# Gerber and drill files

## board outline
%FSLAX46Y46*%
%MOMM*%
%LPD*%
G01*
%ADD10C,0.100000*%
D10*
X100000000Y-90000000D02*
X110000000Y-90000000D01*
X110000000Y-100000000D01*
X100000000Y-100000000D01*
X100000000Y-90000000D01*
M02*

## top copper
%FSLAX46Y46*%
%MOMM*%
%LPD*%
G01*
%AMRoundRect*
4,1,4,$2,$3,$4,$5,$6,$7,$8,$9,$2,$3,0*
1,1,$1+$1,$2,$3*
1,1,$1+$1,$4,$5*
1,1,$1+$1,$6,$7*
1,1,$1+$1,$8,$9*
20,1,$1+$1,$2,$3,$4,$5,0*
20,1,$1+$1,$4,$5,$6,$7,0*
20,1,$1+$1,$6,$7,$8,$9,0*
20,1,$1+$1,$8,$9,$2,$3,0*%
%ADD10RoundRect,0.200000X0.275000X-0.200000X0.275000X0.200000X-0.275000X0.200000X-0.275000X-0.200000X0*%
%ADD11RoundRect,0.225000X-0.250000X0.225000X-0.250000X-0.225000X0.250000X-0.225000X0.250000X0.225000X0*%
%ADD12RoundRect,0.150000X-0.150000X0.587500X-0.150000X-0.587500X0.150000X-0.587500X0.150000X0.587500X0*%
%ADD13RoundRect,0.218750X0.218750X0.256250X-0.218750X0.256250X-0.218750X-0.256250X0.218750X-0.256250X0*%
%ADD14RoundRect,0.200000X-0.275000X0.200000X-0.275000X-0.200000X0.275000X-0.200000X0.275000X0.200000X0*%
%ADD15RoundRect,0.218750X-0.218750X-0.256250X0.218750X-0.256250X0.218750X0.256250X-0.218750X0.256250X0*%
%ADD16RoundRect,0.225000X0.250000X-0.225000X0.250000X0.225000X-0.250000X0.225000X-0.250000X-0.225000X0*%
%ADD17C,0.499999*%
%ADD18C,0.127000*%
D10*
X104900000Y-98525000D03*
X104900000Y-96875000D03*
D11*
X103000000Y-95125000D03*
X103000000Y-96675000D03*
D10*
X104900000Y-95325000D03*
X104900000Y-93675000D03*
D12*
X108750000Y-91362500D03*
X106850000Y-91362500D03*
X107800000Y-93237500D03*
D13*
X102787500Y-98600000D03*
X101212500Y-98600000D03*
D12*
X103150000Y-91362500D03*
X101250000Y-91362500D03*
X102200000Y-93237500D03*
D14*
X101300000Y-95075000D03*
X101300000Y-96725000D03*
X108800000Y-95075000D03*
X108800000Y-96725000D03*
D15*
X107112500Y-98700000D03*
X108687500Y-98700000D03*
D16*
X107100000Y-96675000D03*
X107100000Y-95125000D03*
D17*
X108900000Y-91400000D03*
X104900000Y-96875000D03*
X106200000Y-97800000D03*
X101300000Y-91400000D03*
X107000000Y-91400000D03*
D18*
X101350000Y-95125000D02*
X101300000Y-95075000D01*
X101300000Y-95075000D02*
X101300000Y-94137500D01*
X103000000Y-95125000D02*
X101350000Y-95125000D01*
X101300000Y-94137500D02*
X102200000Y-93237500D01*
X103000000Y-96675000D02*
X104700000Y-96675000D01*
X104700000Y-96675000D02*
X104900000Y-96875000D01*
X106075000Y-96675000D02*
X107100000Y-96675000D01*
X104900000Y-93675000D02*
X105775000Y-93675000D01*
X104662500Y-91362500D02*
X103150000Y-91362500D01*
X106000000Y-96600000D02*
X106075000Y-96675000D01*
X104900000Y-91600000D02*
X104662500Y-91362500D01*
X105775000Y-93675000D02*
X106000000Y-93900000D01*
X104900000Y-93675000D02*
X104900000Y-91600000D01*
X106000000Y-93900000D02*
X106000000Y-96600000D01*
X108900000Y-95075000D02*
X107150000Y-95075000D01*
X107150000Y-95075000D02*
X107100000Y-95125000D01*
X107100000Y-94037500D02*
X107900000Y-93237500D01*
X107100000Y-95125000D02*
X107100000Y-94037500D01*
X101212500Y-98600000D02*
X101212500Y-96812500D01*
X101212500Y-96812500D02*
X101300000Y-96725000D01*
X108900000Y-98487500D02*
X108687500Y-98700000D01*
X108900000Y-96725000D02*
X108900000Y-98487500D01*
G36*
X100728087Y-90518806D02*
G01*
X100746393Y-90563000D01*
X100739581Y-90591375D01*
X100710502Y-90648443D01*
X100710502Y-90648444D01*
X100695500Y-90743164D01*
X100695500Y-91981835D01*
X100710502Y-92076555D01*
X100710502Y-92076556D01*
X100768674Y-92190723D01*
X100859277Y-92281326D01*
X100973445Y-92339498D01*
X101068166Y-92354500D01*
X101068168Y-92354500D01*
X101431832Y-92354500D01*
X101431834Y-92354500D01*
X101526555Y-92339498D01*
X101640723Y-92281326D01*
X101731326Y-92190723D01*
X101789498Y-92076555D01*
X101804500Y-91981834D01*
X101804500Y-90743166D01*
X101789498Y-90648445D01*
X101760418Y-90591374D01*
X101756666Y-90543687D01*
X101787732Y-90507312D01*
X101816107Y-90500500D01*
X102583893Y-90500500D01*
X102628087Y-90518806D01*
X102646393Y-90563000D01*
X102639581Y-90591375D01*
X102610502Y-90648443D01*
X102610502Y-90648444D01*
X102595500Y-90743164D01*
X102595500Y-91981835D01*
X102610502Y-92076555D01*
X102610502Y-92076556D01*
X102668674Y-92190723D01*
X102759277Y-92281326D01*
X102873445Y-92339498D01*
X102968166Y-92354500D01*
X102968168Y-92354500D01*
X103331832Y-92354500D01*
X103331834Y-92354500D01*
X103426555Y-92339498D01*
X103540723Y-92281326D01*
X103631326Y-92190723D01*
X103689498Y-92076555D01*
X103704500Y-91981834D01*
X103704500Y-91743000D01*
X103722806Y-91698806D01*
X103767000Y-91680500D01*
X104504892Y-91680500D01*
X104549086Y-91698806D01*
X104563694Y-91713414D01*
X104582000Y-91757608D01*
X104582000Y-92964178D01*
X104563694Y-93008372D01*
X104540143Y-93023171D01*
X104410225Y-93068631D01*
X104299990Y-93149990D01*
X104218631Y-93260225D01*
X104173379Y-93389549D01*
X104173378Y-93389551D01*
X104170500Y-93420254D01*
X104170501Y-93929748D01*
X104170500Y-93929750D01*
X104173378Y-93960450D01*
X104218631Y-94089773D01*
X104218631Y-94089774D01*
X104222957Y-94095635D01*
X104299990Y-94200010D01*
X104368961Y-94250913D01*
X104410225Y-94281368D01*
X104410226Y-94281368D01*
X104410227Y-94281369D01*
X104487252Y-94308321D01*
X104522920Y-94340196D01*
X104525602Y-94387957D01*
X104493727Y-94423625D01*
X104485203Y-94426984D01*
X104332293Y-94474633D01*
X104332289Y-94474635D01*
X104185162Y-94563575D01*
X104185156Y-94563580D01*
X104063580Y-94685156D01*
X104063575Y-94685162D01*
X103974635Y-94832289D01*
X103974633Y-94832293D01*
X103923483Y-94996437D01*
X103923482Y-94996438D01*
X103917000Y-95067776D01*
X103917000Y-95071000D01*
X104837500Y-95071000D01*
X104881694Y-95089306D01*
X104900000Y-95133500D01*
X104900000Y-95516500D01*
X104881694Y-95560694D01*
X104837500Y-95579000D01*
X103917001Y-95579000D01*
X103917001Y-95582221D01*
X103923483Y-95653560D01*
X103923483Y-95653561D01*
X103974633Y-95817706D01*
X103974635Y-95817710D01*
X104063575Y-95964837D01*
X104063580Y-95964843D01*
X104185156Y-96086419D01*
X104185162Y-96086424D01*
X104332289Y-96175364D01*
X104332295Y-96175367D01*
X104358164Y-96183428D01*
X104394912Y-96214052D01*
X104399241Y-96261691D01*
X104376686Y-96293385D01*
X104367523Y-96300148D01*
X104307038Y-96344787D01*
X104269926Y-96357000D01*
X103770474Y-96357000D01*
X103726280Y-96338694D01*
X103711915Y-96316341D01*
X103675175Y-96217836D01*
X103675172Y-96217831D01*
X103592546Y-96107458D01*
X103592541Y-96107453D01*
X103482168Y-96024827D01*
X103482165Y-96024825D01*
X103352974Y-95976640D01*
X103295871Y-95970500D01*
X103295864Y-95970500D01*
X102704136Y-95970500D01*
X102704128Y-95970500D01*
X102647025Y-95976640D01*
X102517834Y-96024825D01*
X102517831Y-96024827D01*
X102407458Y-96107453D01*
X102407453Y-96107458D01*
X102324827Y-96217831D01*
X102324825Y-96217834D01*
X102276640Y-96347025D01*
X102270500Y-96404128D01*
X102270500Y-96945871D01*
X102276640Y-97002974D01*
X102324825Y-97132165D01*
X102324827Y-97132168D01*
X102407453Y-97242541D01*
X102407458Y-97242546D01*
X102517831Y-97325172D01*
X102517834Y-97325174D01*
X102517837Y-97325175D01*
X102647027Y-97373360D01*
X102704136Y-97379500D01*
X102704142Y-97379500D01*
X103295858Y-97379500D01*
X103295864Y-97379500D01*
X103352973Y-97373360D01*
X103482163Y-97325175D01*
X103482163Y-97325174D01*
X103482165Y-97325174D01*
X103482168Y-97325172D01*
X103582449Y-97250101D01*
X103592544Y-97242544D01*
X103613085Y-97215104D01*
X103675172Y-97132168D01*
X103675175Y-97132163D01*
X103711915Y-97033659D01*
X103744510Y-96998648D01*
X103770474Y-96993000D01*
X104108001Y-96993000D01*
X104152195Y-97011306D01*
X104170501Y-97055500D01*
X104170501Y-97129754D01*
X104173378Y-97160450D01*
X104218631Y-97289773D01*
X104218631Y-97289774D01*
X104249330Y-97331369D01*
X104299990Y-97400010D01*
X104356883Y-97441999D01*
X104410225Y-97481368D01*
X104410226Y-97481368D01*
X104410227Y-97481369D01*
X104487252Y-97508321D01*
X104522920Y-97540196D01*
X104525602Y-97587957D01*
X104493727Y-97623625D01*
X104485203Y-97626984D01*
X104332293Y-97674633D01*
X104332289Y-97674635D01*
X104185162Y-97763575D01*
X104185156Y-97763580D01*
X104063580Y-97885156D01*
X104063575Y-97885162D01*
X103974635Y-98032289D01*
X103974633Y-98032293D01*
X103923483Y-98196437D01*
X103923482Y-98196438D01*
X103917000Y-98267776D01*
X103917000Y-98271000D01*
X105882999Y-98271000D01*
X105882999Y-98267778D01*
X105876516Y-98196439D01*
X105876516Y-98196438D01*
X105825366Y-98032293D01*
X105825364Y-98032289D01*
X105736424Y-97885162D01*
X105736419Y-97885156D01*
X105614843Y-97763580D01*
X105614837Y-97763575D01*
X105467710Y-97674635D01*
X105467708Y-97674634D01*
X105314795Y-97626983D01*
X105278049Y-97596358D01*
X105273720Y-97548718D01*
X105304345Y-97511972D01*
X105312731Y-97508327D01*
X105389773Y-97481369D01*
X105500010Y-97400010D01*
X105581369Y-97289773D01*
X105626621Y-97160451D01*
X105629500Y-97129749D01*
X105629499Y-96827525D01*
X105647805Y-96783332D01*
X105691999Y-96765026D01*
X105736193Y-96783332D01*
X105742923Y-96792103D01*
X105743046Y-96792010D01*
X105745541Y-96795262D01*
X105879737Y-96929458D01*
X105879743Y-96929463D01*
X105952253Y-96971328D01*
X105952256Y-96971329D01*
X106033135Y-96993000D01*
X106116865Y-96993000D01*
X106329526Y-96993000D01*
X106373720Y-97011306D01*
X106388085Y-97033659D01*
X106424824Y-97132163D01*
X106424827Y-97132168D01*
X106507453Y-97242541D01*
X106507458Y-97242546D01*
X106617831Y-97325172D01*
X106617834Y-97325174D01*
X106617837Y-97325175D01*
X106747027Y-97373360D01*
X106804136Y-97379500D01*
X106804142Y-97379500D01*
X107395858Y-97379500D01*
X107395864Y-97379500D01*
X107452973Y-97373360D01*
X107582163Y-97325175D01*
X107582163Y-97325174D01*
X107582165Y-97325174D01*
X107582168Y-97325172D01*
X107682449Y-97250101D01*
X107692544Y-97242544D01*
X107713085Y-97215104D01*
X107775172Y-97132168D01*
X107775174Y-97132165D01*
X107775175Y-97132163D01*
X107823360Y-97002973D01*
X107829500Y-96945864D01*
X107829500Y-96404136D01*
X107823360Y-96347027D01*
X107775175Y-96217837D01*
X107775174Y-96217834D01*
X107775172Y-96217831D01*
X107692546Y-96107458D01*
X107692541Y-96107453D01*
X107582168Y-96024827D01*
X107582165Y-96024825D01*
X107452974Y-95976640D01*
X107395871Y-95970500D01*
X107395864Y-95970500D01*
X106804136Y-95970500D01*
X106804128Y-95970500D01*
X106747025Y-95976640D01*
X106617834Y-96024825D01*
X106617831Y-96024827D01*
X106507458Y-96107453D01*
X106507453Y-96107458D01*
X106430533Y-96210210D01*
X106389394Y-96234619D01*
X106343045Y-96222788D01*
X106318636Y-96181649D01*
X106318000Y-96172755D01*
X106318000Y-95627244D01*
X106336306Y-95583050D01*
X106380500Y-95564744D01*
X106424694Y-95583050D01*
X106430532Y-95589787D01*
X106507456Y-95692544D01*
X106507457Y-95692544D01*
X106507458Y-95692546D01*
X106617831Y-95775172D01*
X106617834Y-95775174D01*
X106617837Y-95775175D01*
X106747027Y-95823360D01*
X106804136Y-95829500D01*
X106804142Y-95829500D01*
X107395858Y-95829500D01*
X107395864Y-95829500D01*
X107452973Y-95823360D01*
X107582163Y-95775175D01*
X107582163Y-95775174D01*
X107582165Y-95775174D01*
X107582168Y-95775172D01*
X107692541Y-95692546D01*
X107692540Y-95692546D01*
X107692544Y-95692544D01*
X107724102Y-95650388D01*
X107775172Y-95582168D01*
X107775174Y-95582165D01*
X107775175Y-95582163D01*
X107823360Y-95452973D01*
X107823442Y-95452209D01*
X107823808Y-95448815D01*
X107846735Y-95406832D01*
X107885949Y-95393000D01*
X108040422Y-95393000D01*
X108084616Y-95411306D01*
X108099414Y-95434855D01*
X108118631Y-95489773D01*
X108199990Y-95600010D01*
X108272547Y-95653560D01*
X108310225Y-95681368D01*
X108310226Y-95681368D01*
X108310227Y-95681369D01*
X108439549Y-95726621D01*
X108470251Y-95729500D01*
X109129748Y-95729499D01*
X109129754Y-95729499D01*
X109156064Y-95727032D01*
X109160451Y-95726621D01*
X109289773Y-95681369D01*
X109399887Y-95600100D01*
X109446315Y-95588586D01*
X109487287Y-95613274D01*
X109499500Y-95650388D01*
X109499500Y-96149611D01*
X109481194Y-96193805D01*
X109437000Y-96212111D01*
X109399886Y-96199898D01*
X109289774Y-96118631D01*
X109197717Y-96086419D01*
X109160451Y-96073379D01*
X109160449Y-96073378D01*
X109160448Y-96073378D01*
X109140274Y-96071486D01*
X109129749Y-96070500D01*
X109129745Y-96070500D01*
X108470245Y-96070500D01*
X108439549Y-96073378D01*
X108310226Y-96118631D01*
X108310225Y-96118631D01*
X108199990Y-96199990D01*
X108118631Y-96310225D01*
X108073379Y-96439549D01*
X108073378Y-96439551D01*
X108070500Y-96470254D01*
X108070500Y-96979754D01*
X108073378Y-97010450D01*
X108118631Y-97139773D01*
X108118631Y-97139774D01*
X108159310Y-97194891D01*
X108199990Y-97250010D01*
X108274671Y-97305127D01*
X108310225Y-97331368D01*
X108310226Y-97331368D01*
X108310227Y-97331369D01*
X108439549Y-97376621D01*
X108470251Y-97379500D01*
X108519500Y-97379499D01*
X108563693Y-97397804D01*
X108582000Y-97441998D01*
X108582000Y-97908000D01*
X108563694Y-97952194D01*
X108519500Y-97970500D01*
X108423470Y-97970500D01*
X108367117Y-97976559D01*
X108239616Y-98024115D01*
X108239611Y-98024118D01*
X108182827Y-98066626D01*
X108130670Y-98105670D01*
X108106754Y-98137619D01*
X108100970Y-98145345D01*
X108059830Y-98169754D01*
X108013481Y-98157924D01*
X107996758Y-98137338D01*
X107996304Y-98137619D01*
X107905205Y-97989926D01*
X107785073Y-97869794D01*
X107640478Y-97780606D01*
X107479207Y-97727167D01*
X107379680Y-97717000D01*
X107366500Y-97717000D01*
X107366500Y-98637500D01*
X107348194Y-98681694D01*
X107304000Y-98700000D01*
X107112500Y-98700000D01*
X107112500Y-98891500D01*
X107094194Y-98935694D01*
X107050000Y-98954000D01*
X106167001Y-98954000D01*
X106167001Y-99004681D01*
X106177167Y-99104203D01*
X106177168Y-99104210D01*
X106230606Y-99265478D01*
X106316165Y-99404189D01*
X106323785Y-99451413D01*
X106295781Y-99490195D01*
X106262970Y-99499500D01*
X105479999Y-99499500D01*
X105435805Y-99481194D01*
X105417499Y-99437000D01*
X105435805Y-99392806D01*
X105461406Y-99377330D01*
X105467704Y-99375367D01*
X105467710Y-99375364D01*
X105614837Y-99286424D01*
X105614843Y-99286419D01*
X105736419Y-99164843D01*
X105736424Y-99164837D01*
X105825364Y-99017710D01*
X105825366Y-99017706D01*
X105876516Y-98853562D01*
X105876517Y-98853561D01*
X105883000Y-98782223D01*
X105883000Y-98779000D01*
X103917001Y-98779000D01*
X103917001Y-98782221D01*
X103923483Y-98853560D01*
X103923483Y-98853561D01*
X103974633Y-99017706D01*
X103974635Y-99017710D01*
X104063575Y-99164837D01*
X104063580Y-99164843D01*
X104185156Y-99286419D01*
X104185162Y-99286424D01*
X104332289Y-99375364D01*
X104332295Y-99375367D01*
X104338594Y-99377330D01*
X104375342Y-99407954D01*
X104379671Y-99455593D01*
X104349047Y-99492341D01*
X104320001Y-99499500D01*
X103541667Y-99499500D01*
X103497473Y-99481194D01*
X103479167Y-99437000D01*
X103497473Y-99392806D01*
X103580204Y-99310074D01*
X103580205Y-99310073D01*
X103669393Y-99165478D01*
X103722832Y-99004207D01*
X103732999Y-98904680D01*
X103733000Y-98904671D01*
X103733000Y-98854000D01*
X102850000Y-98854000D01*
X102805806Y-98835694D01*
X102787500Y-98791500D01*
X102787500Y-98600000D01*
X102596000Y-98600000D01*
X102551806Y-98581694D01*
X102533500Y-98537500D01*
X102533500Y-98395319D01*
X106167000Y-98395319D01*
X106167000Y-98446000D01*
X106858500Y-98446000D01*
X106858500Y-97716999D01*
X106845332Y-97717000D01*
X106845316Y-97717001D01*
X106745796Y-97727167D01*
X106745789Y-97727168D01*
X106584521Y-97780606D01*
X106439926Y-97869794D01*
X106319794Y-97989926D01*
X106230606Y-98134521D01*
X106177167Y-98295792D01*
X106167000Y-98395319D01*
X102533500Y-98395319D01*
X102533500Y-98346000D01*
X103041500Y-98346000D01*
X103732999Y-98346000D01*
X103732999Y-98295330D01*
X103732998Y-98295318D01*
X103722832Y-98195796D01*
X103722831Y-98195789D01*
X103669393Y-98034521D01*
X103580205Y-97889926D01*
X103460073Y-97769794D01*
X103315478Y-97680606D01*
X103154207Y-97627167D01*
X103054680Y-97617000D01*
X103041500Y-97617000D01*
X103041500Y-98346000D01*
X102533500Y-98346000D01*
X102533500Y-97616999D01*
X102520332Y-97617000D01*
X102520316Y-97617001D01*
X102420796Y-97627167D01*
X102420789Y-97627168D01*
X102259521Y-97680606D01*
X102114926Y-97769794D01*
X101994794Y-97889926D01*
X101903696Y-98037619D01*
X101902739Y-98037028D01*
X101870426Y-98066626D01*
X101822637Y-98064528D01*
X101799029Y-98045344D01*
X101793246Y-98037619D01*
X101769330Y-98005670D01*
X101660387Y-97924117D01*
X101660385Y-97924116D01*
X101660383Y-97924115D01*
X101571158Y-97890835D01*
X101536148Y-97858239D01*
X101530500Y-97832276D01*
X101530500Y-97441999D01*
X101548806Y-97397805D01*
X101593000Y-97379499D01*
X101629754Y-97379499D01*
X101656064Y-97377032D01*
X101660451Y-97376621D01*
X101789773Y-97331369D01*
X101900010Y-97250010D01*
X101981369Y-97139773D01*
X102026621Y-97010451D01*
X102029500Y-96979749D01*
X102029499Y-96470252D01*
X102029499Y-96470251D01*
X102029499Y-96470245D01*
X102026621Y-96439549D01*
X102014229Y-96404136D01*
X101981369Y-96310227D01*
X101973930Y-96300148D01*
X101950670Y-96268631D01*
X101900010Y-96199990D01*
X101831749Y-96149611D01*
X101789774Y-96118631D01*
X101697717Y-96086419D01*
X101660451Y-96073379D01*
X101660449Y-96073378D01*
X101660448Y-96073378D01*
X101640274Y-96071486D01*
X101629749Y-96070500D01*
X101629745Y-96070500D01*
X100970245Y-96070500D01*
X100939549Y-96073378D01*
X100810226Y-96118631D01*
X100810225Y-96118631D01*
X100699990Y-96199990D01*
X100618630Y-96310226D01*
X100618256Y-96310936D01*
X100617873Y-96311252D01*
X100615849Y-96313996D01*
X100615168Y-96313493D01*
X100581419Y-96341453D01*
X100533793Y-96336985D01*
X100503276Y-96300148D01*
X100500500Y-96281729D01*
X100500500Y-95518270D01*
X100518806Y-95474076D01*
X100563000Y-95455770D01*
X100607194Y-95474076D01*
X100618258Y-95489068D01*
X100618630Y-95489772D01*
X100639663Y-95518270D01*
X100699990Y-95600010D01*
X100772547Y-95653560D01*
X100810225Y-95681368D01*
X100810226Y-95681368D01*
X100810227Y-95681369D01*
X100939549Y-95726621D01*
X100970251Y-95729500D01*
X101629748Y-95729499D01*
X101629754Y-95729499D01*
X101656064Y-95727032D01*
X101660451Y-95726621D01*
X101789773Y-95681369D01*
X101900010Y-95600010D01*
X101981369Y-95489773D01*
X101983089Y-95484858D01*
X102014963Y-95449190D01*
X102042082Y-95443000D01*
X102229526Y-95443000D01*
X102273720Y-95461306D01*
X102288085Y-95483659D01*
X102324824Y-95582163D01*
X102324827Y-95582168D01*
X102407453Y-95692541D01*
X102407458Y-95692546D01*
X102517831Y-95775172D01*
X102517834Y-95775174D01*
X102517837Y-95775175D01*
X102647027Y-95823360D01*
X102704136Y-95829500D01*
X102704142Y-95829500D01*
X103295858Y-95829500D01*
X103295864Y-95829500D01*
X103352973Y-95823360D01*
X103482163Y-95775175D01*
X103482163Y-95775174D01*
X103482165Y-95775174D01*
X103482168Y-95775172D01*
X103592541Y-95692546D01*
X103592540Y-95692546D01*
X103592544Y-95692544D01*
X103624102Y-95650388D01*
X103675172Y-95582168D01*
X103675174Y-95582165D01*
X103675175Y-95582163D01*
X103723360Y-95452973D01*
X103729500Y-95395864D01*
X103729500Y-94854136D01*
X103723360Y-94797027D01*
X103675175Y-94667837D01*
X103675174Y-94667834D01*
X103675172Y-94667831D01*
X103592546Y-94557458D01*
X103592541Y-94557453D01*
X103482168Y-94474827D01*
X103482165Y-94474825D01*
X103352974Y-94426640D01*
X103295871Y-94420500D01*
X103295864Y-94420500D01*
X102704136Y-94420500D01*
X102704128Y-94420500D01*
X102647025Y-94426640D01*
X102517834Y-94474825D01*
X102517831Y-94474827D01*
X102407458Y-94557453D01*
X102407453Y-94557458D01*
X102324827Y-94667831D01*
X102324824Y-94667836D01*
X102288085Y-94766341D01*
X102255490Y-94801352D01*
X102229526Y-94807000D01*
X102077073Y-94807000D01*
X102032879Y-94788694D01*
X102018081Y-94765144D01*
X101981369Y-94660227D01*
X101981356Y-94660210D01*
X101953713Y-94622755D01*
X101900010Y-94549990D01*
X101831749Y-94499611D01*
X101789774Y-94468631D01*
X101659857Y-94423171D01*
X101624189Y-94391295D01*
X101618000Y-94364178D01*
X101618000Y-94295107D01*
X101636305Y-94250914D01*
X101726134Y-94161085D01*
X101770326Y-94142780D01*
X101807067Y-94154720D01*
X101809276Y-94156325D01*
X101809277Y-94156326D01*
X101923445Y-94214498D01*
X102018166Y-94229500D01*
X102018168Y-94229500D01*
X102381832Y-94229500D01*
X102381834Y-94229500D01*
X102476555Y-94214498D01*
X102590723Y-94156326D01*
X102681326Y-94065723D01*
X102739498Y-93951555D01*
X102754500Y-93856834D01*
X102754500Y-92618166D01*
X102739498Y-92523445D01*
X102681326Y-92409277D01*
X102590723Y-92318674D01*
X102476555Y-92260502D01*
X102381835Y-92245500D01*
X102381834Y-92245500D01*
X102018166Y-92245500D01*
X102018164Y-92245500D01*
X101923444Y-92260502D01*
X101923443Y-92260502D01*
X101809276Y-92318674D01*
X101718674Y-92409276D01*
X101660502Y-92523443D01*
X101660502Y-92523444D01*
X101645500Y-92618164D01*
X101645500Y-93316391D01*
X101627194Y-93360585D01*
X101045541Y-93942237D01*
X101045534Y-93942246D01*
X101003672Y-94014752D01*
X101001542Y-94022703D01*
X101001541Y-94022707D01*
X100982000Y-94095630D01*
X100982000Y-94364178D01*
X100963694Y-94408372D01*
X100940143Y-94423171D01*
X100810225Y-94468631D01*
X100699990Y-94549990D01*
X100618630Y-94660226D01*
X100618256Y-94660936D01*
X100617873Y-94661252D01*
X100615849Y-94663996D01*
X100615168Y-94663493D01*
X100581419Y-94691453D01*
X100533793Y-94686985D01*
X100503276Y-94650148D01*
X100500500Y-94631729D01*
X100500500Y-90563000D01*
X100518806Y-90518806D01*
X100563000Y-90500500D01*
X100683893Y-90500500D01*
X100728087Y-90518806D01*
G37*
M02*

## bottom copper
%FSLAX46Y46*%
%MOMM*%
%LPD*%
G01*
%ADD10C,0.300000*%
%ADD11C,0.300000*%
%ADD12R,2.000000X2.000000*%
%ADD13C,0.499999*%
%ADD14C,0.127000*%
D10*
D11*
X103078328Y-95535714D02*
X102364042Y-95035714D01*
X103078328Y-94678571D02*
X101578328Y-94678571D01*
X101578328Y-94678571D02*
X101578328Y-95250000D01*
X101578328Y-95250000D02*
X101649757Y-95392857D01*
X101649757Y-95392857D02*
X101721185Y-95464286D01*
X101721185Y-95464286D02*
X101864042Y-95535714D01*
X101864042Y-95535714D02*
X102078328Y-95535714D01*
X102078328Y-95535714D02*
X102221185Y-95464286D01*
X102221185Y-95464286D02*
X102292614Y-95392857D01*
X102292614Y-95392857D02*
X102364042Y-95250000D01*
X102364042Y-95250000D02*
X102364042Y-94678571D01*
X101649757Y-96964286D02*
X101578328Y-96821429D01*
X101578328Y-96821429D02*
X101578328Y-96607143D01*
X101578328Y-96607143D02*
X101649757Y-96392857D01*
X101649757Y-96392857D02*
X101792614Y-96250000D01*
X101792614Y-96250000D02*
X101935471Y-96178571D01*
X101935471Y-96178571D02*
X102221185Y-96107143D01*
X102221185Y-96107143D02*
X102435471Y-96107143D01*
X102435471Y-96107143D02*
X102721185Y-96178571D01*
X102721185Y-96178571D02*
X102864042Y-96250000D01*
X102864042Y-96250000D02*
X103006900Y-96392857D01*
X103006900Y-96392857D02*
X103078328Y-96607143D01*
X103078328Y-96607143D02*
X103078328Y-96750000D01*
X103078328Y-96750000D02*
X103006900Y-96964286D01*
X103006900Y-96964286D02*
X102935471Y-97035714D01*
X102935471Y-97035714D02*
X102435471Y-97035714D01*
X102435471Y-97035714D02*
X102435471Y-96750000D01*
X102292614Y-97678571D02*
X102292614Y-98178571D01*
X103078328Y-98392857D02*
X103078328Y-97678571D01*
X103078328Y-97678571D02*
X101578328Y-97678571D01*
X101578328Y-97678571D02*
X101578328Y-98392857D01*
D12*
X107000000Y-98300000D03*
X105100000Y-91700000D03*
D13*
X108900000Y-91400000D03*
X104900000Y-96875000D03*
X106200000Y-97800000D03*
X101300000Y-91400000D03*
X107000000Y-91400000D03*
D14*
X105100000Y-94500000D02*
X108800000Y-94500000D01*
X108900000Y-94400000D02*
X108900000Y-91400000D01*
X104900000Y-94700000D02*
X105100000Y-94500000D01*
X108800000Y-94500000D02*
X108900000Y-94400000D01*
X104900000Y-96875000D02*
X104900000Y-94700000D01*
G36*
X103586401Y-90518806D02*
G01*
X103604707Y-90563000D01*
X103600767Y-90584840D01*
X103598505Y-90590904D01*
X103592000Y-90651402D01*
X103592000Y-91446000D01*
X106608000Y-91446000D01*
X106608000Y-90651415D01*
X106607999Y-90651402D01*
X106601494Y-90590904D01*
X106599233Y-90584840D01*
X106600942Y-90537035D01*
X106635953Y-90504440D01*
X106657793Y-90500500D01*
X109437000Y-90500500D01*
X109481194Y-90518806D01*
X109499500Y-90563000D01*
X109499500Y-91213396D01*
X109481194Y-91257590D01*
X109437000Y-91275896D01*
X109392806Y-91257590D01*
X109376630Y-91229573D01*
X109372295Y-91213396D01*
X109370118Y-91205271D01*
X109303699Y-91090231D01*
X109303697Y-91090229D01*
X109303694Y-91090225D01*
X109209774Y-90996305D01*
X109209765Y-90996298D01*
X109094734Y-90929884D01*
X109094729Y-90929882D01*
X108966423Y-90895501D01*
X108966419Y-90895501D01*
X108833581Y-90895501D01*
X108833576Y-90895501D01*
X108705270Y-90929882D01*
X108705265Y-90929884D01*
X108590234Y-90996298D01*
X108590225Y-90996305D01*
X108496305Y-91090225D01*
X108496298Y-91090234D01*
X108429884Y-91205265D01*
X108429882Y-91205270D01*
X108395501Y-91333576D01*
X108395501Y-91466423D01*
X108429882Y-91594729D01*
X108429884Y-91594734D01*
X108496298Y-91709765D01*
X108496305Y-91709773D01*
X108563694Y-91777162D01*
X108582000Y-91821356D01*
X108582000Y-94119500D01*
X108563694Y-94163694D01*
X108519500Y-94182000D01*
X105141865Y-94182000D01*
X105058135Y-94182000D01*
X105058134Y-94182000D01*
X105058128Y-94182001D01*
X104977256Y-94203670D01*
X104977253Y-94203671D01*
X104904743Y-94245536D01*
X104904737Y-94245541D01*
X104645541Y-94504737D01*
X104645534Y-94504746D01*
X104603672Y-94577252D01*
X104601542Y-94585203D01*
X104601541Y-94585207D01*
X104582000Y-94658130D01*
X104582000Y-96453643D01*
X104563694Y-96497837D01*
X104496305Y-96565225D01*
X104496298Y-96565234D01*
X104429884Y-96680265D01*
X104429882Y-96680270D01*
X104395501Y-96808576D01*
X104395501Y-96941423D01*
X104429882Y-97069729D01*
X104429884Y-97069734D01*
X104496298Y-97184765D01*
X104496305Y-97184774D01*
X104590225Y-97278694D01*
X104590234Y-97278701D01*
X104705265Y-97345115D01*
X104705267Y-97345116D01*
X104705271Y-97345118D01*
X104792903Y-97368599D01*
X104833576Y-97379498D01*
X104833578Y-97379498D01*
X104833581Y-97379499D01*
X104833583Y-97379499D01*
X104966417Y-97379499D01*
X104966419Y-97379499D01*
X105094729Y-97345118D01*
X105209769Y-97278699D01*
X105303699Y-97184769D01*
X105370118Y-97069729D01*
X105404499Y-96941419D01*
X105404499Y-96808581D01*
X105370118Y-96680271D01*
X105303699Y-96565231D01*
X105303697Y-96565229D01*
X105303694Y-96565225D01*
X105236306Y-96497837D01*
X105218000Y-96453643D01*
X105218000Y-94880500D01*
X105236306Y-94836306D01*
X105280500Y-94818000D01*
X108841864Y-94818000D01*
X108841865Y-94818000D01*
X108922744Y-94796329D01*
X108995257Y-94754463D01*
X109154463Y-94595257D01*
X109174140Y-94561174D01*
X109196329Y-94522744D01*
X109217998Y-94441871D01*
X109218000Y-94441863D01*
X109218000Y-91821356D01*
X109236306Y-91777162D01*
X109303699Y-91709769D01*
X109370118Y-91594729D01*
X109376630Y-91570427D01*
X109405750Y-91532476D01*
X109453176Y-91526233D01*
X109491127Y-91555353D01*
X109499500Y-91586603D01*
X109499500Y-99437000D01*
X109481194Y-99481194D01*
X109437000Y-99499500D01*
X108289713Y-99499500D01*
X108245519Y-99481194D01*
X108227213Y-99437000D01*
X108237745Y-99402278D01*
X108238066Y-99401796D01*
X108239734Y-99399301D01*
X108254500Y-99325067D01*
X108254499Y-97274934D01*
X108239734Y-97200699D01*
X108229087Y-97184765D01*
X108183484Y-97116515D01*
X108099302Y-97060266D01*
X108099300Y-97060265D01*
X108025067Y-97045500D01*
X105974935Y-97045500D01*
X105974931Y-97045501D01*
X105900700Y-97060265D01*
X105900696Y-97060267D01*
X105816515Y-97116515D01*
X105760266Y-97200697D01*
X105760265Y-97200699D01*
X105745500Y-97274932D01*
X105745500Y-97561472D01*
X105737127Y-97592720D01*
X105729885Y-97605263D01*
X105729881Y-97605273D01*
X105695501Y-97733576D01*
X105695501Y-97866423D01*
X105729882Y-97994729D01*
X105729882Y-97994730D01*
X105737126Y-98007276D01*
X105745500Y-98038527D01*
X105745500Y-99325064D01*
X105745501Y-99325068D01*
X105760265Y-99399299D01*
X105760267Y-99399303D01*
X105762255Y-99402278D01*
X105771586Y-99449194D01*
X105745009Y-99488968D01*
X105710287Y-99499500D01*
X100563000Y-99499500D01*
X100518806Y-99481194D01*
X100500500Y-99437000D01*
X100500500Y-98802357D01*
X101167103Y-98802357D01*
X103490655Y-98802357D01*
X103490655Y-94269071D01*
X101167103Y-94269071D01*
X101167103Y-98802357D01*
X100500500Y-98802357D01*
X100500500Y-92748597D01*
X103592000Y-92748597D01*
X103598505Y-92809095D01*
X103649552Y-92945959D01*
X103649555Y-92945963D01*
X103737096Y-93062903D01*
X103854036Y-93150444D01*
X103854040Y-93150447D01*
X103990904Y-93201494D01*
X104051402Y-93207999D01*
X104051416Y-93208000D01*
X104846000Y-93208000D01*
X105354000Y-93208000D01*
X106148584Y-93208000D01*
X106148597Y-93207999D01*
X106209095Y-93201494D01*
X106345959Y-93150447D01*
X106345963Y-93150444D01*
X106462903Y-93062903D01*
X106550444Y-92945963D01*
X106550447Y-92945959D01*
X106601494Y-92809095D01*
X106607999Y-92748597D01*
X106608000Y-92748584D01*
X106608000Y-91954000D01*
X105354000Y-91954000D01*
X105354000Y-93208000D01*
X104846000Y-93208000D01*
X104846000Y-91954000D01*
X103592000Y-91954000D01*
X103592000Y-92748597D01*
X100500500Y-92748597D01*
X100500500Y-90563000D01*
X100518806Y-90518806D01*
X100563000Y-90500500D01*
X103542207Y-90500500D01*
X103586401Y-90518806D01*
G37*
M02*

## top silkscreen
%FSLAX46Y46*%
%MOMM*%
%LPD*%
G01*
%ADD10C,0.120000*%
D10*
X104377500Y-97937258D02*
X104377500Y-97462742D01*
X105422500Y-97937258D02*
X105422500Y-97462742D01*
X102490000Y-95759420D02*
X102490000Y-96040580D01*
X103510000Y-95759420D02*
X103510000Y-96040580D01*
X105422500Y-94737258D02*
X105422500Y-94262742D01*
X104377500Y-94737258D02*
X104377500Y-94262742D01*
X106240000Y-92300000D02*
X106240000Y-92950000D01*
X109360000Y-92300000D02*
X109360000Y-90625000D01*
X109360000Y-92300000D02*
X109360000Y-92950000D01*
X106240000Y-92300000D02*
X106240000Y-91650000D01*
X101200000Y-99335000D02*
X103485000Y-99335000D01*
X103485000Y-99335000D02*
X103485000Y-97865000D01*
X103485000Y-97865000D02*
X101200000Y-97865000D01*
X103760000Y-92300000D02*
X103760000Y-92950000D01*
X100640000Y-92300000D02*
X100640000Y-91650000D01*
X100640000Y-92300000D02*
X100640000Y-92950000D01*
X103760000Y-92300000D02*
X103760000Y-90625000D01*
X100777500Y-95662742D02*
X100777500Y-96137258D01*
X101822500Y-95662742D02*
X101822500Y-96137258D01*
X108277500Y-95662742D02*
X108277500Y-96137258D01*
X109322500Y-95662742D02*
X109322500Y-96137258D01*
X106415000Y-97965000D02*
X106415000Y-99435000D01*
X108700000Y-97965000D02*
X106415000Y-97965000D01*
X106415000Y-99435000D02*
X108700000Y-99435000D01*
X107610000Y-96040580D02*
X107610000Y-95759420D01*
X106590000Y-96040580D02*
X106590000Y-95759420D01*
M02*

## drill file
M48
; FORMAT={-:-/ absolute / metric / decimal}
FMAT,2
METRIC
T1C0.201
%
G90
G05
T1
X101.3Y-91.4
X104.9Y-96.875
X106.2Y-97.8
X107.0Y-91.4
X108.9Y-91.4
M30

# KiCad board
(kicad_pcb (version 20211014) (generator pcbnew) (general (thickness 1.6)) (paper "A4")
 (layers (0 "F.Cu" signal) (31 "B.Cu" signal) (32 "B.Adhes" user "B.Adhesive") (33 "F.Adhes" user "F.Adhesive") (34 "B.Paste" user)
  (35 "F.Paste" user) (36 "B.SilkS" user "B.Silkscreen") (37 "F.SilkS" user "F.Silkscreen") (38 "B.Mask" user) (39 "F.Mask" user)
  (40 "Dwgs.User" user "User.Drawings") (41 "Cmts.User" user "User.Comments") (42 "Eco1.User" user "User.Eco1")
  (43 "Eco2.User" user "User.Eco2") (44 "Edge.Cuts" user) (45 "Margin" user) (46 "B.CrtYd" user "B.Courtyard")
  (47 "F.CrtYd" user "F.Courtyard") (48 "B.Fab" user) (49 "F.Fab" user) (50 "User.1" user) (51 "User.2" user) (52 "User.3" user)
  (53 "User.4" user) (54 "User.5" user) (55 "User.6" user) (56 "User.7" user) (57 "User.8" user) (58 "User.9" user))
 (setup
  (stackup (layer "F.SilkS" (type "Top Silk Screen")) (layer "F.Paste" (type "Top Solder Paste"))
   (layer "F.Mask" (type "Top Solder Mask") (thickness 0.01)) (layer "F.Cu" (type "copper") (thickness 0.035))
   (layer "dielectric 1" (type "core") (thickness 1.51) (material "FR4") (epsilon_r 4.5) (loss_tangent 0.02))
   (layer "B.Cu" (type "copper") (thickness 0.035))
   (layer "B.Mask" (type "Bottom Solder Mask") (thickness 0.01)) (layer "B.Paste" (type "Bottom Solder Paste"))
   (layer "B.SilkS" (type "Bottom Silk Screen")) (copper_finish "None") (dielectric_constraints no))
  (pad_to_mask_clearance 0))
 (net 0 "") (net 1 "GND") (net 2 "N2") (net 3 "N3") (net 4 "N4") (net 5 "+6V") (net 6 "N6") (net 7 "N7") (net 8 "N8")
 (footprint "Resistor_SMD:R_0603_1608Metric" (layer "F.Cu") (at 104.9 97.7 90)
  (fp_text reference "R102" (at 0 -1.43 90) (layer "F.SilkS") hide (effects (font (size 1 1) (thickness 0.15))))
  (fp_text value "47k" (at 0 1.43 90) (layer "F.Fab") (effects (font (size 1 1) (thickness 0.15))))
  (fp_line (start -0.237258 -0.5225) (end 0.237258 -0.5225) (layer "F.SilkS") (width 0.12))
  (fp_line (start -0.237258 0.5225) (end 0.237258 0.5225) (layer "F.SilkS") (width 0.12))
  (pad "1" smd roundrect (at -0.825 0 90) (size 0.8 0.95) (layers "F.Cu" "F.Paste" "F.Mask") (roundrect_rratio 0.25) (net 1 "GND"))
  (pad "2" smd roundrect (at 0.825 0 90) (size 0.8 0.95) (layers "F.Cu" "F.Paste" "F.Mask") (roundrect_rratio 0.25) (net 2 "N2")))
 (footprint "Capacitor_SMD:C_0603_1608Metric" (layer "F.Cu") (at 103 95.9 -90)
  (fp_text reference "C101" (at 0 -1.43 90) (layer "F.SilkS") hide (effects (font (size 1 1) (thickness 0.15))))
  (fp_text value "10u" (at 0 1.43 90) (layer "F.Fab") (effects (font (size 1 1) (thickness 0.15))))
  (fp_line (start -0.14058 0.51) (end 0.14058 0.51) (layer "F.SilkS") (width 0.12))
  (fp_line (start -0.14058 -0.51) (end 0.14058 -0.51) (layer "F.SilkS") (width 0.12))
  (pad "1" smd roundrect (at -0.775 0 270) (size 0.9 0.95) (layers "F.Cu" "F.Paste" "F.Mask") (roundrect_rratio 0.25) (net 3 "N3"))
  (pad "2" smd roundrect (at 0.775 0 270) (size 0.9 0.95) (layers "F.Cu" "F.Paste" "F.Mask") (roundrect_rratio 0.25) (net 2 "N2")))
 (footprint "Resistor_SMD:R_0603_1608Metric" (layer "F.Cu") (at 104.9 94.5 90)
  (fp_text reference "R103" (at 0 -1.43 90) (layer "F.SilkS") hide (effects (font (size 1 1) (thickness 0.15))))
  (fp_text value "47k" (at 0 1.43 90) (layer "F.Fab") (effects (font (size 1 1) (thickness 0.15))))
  (fp_line (start -0.237258 0.5225) (end 0.237258 0.5225) (layer "F.SilkS") (width 0.12))
  (fp_line (start -0.237258 -0.5225) (end 0.237258 -0.5225) (layer "F.SilkS") (width 0.12))
  (pad "1" smd roundrect (at -0.825 0 90) (size 0.8 0.95) (layers "F.Cu" "F.Paste" "F.Mask") (roundrect_rratio 0.25) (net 1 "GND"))
  (pad "2" smd roundrect (at 0.825 0 90) (size 0.8 0.95) (layers "F.Cu" "F.Paste" "F.Mask") (roundrect_rratio 0.25) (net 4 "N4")))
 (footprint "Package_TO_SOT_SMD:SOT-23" (layer "F.Cu") (at 107.8 92.3 -90)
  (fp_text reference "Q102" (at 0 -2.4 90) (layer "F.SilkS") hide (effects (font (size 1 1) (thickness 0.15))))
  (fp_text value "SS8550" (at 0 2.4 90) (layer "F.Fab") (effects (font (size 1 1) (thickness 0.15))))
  (fp_line (start 0 1.56) (end 0.65 1.56) (layer "F.SilkS") (width 0.12))
  (fp_line (start 0 -1.56) (end -1.675 -1.56) (layer "F.SilkS") (width 0.12))
  (fp_line (start 0 -1.56) (end 0.65 -1.56) (layer "F.SilkS") (width 0.12))
  (fp_line (start 0 1.56) (end -0.65 1.56) (layer "F.SilkS") (width 0.12))
  (pad "1" smd roundrect (at -0.9375 -0.95 270) (size 1.475 0.6) (layers "F.Cu" "F.Paste" "F.Mask") (roundrect_rratio 0.25) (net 2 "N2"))
  (pad "2" smd roundrect (at -0.9375 0.95 270) (size 1.475 0.6) (layers "F.Cu" "F.Paste" "F.Mask") (roundrect_rratio 0.25) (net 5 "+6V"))
  (pad "3" smd roundrect (at 0.9375 0 270) (size 1.475 0.6) (layers "F.Cu" "F.Paste" "F.Mask") (roundrect_rratio 0.25) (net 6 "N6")))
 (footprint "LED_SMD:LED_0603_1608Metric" (layer "F.Cu") (at 102 98.6 180)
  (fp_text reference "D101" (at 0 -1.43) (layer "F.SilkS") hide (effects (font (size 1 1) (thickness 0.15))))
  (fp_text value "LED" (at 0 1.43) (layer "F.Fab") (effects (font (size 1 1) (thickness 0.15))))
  (fp_line (start 0.8 -0.735) (end -1.485 -0.735) (layer "F.SilkS") (width 0.12))
  (fp_line (start -1.485 -0.735) (end -1.485 0.735) (layer "F.SilkS") (width 0.12))
  (fp_line (start -1.485 0.735) (end 0.8 0.735) (layer "F.SilkS") (width 0.12))
  (pad "1" smd roundrect (at -0.7875 0 180) (size 0.875 0.95) (layers "F.Cu" "F.Paste" "F.Mask") (roundrect_rratio 0.25) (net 1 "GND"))
  (pad "2" smd roundrect (at 0.7875 0 180) (size 0.875 0.95) (layers "F.Cu" "F.Paste" "F.Mask") (roundrect_rratio 0.25) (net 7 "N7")))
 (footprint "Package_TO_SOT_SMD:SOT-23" (layer "F.Cu") (at 102.2 92.3 -90)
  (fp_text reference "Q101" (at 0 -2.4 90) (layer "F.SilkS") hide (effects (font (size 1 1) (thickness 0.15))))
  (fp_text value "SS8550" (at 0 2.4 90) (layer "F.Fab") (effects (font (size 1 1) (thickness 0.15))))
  (fp_line (start 0 -1.56) (end 0.65 -1.56) (layer "F.SilkS") (width 0.12))
  (fp_line (start 0 1.56) (end -0.65 1.56) (layer "F.SilkS") (width 0.12))
  (fp_line (start 0 1.56) (end 0.65 1.56) (layer "F.SilkS") (width 0.12))
  (fp_line (start 0 -1.56) (end -1.675 -1.56) (layer "F.SilkS") (width 0.12))
  (pad "1" smd roundrect (at -0.9375 -0.95 270) (size 1.475 0.6) (layers "F.Cu" "F.Paste" "F.Mask") (roundrect_rratio 0.25) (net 4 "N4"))
  (pad "2" smd roundrect (at -0.9375 0.95 270) (size 1.475 0.6) (layers "F.Cu" "F.Paste" "F.Mask") (roundrect_rratio 0.25) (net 5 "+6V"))
  (pad "3" smd roundrect (at 0.9375 0 270) (size 1.475 0.6) (layers "F.Cu" "F.Paste" "F.Mask") (roundrect_rratio 0.25) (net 3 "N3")))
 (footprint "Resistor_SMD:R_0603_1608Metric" (layer "F.Cu") (at 101.3 95.9 -90)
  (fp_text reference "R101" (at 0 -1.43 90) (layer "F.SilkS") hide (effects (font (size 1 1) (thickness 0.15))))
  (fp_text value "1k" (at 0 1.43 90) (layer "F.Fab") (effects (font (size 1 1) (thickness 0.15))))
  (fp_line (start -0.237258 0.5225) (end 0.237258 0.5225) (layer "F.SilkS") (width 0.12))
  (fp_line (start -0.237258 -0.5225) (end 0.237258 -0.5225) (layer "F.SilkS") (width 0.12))
  (pad "1" smd roundrect (at -0.825 0 270) (size 0.8 0.95) (layers "F.Cu" "F.Paste" "F.Mask") (roundrect_rratio 0.25) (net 3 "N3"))
  (pad "2" smd roundrect (at 0.825 0 270) (size 0.8 0.95) (layers "F.Cu" "F.Paste" "F.Mask") (roundrect_rratio 0.25) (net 7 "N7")))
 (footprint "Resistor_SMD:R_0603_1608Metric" (layer "F.Cu") (at 108.8 95.9 -90)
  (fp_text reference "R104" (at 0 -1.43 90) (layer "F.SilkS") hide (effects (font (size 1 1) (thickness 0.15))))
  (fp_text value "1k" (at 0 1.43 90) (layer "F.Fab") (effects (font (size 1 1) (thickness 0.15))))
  (fp_line (start -0.237258 0.5225) (end 0.237258 0.5225) (layer "F.SilkS") (width 0.12))
  (fp_line (start -0.237258 -0.5225) (end 0.237258 -0.5225) (layer "F.SilkS") (width 0.12))
  (pad "1" smd roundrect (at -0.825 0 270) (size 0.8 0.95) (layers "F.Cu" "F.Paste" "F.Mask") (roundrect_rratio 0.25) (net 6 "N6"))
  (pad "2" smd roundrect (at 0.825 0 270) (size 0.8 0.95) (layers "F.Cu" "F.Paste" "F.Mask") (roundrect_rratio 0.25) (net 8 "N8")))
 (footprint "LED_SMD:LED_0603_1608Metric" (layer "F.Cu") (at 107.9 98.7)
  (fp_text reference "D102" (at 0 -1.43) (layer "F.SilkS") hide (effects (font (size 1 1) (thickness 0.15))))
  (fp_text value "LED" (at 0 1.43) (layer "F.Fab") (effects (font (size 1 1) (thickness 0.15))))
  (fp_line (start -1.485 -0.735) (end -1.485 0.735) (layer "F.SilkS") (width 0.12))
  (fp_line (start 0.8 -0.735) (end -1.485 -0.735) (layer "F.SilkS") (width 0.12))
  (fp_line (start -1.485 0.735) (end 0.8 0.735) (layer "F.SilkS") (width 0.12))
  (pad "1" smd roundrect (at -0.7875 0) (size 0.875 0.95) (layers "F.Cu" "F.Paste" "F.Mask") (roundrect_rratio 0.25) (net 1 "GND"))
  (pad "2" smd roundrect (at 0.7875 0) (size 0.875 0.95) (layers "F.Cu" "F.Paste" "F.Mask") (roundrect_rratio 0.25) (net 8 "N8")))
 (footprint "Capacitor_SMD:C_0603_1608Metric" (layer "F.Cu") (at 107.1 95.9 90)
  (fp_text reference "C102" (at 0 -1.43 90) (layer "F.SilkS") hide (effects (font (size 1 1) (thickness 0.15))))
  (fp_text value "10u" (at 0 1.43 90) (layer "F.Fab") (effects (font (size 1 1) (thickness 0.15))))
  (fp_line (start -0.14058 0.51) (end 0.14058 0.51) (layer "F.SilkS") (width 0.12))
  (fp_line (start -0.14058 -0.51) (end 0.14058 -0.51) (layer "F.SilkS") (width 0.12))
  (pad "1" smd roundrect (at -0.775 0 90) (size 0.9 0.95) (layers "F.Cu" "F.Paste" "F.Mask") (roundrect_rratio 0.25) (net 4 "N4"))
  (pad "2" smd roundrect (at 0.775 0 90) (size 0.9 0.95) (layers "F.Cu" "F.Paste" "F.Mask") (roundrect_rratio 0.25) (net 6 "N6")))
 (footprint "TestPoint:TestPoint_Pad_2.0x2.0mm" (layer "B.Cu") (at 107 98.3 180)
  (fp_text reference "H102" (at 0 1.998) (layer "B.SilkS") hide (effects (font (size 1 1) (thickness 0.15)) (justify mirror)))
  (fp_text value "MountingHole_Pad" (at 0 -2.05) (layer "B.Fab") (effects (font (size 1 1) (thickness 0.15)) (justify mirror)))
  (pad "1" smd rect (at 0 0 180) (size 2 2) (layers "B.Cu" "B.Mask") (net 1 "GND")))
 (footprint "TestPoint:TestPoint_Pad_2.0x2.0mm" (layer "B.Cu") (at 105.1 91.7 180)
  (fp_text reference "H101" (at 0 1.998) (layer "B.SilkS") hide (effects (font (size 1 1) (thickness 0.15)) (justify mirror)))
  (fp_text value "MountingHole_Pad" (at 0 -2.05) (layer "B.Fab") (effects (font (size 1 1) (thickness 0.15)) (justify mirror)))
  (pad "1" smd rect (at 0 0 180) (size 2 2) (layers "B.Cu" "B.Mask") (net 5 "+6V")))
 (gr_rect (start 100 90) (end 110 100) (layer "Edge.Cuts") (width 0.1) (fill none))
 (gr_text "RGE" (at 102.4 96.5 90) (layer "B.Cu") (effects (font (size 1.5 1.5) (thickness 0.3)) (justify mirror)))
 (segment (start 101.35 95.125) (end 101.3 95.075) (width 0.127) (layer "F.Cu") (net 3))
 (segment (start 101.3 95.075) (end 101.3 94.1375) (width 0.127) (layer "F.Cu") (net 3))
 (segment (start 103 95.125) (end 101.35 95.125) (width 0.127) (layer "F.Cu") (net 3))
 (segment (start 101.3 94.1375) (end 102.2 93.2375) (width 0.127) (layer "F.Cu") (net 3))
 (segment (start 103 96.675) (end 104.7 96.675) (width 0.127) (layer "F.Cu") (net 2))
 (segment (start 104.7 96.675) (end 104.9 96.875) (width 0.127) (layer "F.Cu") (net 2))
 (via (at 108.9 91.4) (size 0.499999) (drill 0.20066) (layers "F.Cu" "B.Cu") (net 2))
 (via (at 104.9 96.875) (size 0.499999) (drill 0.20066) (layers "F.Cu" "B.Cu") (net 2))
 (segment (start 105.1 94.5) (end 108.8 94.5) (width 0.127) (layer "B.Cu") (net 2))
 (segment (start 108.9 94.4) (end 108.9 91.4) (width 0.127) (layer "B.Cu") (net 2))
 (segment (start 104.9 94.7) (end 105.1 94.5) (width 0.127) (layer "B.Cu") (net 2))
 (segment (start 108.8 94.5) (end 108.9 94.4) (width 0.127) (layer "B.Cu") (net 2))
 (segment (start 104.9 96.875) (end 104.9 94.7) (width 0.127) (layer "B.Cu") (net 2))
 (segment (start 106.075 96.675) (end 107.1 96.675) (width 0.127) (layer "F.Cu") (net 4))
 (segment (start 104.9 93.675) (end 105.775 93.675) (width 0.127) (layer "F.Cu") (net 4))
 (segment (start 104.6625 91.3625) (end 103.15 91.3625) (width 0.127) (layer "F.Cu") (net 4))
 (segment (start 106 96.6) (end 106.075 96.675) (width 0.127) (layer "F.Cu") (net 4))
 (segment (start 104.9 91.6) (end 104.6625 91.3625) (width 0.127) (layer "F.Cu") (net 4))
 (segment (start 105.775 93.675) (end 106 93.9) (width 0.127) (layer "F.Cu") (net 4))
 (segment (start 104.9 93.675) (end 104.9 91.6) (width 0.127) (layer "F.Cu") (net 4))
 (segment (start 106 93.9) (end 106 96.6) (width 0.127) (layer "F.Cu") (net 4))
 (segment (start 108.9 95.075) (end 107.15 95.075) (width 0.127) (layer "F.Cu") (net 6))
 (segment (start 107.15 95.075) (end 107.1 95.125) (width 0.127) (layer "F.Cu") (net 6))
 (segment (start 107.1 94.0375) (end 107.9 93.2375) (width 0.127) (layer "F.Cu") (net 6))
 (segment (start 107.1 95.125) (end 107.1 94.0375) (width 0.127) (layer "F.Cu") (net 6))
 (via (at 106.2 97.8) (size 0.499999) (drill 0.20066) (layers "F.Cu" "B.Cu") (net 1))
 (segment (start 101.2125 98.6) (end 101.2125 96.8125) (width 0.127) (layer "F.Cu") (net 7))
 (segment (start 101.2125 96.8125) (end 101.3 96.725) (width 0.127) (layer "F.Cu") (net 7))
 (segment (start 108.9 98.4875) (end 108.6875 98.7) (width 0.127) (layer "F.Cu") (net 8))
 (segment (start 108.9 96.725) (end 108.9 98.4875) (width 0.127) (layer "F.Cu") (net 8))
 (via (at 101.3 91.4) (size 0.499999) (drill 0.20066) (layers "F.Cu" "B.Cu") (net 5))
 (via (at 107 91.4) (size 0.499999) (drill 0.20066) (layers "F.Cu" "B.Cu") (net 5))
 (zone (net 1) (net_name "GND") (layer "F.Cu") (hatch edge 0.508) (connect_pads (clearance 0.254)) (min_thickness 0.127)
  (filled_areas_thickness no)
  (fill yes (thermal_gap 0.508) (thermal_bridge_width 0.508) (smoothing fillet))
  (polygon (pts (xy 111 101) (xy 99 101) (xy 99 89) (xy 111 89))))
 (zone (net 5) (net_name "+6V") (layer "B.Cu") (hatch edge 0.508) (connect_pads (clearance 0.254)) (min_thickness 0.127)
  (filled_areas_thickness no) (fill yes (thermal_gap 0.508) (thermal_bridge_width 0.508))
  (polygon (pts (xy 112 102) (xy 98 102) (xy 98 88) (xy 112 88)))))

